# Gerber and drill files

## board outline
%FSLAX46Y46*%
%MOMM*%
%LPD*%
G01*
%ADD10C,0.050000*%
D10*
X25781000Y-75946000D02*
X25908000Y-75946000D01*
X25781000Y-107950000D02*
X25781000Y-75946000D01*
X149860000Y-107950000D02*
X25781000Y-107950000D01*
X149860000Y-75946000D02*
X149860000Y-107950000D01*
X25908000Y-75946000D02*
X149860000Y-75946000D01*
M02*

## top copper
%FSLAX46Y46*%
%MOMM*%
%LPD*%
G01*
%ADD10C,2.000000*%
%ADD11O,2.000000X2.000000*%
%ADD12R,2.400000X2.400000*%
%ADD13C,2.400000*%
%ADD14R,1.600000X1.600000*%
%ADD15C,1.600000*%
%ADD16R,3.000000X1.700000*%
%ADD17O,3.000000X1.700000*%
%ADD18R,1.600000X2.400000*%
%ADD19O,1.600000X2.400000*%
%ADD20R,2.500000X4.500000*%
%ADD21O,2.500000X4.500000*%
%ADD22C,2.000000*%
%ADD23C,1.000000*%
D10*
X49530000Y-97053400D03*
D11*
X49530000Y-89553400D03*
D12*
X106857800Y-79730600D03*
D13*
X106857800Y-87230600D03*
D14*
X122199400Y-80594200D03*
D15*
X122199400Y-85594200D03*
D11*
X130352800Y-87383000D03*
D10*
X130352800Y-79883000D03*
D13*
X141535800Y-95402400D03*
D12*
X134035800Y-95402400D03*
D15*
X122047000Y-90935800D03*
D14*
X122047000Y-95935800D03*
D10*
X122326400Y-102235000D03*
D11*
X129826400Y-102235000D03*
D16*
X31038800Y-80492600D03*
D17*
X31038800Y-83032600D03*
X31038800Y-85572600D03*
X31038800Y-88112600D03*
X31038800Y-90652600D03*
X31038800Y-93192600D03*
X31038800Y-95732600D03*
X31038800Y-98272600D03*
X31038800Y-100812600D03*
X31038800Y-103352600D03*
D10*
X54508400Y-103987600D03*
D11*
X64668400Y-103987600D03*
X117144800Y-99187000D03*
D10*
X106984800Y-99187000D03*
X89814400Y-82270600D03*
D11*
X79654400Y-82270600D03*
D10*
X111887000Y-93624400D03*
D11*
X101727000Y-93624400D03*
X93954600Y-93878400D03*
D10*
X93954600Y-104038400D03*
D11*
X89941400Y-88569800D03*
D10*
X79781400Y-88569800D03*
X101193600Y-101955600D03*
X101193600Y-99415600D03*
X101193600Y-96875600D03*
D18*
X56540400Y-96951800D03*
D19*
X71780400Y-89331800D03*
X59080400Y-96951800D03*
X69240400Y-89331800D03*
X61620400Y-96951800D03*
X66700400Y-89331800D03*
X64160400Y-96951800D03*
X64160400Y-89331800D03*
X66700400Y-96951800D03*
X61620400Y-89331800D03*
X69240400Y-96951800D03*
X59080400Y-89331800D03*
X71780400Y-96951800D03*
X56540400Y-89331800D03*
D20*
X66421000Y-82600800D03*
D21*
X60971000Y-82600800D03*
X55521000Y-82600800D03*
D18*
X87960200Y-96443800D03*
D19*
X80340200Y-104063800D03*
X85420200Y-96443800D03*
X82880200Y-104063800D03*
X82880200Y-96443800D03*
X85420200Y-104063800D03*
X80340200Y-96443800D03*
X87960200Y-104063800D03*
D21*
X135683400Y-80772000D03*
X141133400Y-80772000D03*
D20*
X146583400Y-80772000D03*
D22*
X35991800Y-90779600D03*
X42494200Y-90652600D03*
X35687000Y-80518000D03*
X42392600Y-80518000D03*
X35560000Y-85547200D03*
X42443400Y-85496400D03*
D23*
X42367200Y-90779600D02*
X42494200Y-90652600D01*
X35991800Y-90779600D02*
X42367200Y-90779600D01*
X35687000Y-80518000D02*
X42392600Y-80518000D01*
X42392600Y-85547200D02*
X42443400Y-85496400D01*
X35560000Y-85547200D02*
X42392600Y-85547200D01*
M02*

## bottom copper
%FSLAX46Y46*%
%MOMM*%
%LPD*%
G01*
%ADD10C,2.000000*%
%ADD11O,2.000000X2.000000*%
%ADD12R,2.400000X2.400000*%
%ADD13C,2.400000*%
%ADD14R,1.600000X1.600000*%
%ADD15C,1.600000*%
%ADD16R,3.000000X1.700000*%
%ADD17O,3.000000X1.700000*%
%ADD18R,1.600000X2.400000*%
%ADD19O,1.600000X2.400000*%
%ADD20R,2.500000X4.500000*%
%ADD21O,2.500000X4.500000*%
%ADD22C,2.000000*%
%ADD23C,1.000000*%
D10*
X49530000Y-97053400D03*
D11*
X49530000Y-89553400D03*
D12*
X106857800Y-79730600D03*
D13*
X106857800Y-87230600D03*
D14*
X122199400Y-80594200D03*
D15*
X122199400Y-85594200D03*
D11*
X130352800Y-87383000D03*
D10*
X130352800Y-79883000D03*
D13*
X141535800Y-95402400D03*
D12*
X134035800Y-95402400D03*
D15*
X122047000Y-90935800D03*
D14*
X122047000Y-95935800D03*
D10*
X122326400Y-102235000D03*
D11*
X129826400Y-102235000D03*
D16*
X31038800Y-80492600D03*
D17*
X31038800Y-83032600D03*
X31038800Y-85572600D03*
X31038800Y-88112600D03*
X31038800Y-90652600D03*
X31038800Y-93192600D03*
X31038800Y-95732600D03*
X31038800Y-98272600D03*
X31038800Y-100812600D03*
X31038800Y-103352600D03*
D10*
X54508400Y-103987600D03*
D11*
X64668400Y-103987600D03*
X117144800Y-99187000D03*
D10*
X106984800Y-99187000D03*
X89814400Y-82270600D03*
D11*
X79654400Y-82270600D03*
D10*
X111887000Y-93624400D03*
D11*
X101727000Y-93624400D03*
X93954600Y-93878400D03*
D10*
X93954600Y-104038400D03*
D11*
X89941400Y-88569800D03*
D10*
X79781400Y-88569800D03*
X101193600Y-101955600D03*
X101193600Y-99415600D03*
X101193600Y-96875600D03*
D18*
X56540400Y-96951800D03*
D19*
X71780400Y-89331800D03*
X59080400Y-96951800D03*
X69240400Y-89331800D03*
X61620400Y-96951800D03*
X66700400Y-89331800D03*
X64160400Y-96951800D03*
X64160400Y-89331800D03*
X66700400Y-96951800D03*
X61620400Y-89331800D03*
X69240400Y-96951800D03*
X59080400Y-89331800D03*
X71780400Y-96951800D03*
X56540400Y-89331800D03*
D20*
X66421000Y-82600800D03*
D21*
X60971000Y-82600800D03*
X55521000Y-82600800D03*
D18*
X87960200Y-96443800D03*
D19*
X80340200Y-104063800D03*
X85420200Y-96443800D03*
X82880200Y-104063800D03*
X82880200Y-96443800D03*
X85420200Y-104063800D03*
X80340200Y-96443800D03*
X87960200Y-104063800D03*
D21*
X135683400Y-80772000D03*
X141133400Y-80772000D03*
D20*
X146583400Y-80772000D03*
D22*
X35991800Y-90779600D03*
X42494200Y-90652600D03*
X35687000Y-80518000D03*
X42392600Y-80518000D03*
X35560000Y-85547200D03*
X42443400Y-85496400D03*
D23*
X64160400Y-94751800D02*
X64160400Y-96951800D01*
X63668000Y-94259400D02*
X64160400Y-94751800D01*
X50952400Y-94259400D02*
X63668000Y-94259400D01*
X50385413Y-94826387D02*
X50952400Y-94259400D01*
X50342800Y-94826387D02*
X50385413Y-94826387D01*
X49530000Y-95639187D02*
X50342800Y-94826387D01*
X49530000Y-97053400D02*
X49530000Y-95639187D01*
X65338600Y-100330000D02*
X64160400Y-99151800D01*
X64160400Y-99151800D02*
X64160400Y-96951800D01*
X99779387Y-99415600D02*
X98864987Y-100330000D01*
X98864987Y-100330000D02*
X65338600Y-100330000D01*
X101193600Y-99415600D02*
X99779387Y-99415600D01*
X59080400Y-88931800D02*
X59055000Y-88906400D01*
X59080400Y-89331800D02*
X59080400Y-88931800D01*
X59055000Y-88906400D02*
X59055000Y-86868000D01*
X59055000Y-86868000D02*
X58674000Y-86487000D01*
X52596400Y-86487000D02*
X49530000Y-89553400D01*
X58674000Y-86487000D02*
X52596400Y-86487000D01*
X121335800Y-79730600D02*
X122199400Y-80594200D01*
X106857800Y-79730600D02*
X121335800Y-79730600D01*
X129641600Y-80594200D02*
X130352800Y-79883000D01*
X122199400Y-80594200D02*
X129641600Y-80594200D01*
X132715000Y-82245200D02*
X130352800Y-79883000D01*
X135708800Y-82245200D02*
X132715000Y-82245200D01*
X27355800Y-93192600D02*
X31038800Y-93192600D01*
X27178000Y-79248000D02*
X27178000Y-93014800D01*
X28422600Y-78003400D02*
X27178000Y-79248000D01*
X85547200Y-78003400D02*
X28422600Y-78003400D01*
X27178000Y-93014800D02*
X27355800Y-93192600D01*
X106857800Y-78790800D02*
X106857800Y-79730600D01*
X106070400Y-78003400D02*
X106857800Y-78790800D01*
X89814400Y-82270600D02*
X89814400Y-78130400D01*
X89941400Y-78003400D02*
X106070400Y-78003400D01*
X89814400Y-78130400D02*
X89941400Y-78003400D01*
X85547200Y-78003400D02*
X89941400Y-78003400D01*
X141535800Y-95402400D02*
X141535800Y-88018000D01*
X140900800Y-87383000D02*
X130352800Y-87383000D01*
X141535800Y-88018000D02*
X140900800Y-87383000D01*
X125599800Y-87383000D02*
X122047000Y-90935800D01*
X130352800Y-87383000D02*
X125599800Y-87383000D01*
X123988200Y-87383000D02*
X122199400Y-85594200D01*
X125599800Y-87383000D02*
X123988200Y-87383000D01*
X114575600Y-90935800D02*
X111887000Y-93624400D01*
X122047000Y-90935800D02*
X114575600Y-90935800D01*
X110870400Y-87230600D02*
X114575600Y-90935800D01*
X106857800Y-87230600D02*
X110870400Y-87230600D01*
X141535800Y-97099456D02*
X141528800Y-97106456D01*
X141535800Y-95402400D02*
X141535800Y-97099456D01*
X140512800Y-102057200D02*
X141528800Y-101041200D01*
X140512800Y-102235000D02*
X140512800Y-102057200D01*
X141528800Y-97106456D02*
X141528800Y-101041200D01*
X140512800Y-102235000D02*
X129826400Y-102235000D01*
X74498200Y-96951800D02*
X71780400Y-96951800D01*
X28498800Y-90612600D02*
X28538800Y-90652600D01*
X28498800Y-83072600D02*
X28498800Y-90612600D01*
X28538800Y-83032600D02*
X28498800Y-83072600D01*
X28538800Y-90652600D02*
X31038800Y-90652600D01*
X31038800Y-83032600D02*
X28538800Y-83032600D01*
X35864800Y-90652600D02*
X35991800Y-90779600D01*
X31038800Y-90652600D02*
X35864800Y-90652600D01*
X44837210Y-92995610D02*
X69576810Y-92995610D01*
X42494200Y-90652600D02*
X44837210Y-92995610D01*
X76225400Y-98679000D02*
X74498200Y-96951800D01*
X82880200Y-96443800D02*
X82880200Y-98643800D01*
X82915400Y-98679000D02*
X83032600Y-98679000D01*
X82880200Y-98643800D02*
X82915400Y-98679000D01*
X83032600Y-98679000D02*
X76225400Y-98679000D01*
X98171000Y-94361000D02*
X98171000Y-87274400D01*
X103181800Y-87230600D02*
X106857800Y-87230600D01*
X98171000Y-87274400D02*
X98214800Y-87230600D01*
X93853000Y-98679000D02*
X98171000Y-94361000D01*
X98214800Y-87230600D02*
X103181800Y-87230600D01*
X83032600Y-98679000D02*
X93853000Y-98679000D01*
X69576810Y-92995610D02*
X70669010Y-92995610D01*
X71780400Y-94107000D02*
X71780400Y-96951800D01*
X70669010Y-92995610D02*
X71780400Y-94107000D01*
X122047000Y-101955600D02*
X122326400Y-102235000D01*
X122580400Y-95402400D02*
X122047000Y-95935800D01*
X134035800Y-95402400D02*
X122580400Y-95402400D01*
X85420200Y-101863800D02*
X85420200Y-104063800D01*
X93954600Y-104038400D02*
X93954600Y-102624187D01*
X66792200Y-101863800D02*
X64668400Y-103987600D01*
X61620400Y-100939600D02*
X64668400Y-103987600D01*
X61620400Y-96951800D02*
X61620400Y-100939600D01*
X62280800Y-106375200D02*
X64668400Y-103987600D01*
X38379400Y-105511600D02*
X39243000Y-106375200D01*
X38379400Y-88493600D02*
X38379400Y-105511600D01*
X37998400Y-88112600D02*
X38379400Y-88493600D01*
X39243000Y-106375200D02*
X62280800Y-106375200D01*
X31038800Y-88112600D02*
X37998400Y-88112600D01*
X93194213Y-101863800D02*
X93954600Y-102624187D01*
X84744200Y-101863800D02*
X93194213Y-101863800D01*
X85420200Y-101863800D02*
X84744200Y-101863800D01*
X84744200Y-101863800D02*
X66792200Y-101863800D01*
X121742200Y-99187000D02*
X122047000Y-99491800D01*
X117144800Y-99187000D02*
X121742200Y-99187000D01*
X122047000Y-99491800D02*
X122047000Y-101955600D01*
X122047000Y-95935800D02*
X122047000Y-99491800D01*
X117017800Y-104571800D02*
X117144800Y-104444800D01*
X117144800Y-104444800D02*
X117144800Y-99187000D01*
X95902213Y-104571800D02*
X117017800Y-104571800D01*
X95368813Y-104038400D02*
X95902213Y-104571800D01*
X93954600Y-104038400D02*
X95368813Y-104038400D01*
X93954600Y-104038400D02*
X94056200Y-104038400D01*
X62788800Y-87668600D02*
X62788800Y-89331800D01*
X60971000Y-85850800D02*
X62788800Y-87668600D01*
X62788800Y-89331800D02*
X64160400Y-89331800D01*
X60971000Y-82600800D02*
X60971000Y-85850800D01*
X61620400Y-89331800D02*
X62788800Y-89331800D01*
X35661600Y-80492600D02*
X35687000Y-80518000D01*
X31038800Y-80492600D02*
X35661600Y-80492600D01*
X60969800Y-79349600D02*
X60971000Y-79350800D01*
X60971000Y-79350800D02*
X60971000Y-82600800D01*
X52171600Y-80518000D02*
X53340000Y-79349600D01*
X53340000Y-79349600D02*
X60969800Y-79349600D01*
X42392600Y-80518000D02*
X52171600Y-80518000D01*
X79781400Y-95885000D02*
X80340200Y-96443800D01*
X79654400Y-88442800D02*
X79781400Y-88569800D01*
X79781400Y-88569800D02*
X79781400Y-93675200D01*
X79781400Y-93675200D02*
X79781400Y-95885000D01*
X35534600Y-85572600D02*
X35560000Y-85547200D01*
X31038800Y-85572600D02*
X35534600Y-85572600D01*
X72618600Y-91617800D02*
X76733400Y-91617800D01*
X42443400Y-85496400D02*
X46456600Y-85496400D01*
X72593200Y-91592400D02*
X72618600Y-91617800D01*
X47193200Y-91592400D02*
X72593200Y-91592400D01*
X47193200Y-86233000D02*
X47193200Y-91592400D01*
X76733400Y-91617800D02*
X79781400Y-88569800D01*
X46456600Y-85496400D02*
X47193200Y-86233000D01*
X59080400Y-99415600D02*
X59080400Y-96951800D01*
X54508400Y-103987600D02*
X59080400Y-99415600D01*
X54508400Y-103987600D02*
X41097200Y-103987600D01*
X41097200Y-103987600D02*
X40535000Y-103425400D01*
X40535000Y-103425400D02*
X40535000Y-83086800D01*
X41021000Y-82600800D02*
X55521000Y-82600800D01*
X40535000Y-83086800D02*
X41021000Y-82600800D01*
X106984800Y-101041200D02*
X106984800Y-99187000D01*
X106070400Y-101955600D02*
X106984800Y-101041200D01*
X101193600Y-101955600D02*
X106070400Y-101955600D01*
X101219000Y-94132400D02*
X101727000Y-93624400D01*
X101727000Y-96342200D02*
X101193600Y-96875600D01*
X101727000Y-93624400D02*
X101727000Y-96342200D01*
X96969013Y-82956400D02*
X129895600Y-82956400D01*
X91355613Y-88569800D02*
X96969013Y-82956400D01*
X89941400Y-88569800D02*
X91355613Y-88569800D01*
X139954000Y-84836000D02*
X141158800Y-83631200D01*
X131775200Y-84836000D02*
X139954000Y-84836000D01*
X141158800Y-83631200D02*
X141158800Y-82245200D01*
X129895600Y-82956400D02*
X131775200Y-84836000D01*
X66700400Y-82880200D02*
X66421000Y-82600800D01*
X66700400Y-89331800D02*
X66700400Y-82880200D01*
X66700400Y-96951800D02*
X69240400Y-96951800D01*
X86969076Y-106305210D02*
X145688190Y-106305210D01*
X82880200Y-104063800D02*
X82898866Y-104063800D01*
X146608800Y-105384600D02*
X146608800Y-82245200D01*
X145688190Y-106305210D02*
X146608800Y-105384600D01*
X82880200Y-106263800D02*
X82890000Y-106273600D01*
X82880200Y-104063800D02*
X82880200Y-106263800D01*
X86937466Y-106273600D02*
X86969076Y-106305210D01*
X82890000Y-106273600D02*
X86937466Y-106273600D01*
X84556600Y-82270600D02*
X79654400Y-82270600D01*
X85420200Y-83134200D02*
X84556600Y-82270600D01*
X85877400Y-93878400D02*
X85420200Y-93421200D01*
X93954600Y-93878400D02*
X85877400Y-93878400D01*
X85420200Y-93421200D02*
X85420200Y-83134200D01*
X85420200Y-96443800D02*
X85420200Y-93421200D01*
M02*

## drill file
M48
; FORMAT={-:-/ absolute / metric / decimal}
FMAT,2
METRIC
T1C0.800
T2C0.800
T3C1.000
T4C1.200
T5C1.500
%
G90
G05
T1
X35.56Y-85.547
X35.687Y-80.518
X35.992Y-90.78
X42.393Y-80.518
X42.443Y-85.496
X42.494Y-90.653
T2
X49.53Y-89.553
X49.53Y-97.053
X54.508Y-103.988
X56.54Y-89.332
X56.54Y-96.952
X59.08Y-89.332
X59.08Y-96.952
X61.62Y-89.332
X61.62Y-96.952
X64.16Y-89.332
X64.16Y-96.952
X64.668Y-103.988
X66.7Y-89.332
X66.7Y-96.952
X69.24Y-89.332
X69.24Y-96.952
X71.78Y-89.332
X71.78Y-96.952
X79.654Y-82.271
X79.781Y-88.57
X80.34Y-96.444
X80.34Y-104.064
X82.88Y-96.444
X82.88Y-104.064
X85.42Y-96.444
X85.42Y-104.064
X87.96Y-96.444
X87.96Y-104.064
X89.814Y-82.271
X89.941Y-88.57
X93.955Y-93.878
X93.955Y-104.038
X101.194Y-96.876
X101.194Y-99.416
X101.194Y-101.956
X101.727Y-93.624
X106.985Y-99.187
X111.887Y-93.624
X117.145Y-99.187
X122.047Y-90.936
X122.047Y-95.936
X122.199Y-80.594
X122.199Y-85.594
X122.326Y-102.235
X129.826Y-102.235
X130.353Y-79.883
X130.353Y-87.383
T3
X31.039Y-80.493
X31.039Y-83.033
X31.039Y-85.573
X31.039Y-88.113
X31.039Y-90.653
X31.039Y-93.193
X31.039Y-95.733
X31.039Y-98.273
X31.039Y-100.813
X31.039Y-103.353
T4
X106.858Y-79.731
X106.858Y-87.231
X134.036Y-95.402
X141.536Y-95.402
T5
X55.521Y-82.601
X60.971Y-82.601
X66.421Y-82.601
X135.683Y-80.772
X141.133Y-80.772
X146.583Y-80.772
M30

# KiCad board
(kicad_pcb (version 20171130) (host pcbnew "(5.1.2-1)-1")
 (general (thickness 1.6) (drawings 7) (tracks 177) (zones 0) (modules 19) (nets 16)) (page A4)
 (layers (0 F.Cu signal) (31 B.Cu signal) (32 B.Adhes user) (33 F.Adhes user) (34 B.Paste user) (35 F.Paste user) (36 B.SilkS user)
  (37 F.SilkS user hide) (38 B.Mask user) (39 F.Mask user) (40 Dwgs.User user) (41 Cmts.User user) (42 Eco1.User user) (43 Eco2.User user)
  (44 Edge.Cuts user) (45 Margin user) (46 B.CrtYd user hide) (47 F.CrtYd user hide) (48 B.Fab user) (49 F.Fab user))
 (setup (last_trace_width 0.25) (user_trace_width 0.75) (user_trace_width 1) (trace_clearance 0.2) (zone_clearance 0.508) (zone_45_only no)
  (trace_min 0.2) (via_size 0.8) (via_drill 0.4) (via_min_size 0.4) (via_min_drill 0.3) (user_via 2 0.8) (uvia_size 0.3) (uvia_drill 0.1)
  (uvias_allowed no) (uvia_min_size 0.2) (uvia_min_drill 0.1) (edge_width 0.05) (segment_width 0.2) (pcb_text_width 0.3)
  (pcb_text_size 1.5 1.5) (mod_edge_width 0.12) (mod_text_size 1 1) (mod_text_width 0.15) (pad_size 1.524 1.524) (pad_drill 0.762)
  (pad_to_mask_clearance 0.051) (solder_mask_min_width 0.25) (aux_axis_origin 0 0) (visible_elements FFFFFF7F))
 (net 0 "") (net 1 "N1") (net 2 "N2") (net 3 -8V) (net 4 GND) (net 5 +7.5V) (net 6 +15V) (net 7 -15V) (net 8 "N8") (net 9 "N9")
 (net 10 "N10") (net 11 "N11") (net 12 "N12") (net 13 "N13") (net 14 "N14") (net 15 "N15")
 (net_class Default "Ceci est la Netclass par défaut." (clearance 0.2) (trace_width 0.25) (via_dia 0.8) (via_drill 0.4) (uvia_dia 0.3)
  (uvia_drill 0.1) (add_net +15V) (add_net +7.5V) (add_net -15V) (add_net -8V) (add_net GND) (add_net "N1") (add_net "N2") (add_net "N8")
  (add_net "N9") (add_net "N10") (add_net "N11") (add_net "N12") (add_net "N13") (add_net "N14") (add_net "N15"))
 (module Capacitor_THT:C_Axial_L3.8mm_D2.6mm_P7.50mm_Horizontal (layer F.Cu) (at 49.53 97.0534 90)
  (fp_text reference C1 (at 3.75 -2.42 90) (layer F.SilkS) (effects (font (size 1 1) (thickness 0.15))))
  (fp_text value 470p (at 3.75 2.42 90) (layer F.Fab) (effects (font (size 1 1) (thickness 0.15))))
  (pad 1 thru_hole circle (at 0 0 90) (size 2 2) (drill 0.8) (layers *.Cu *.Mask) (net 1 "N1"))
  (pad 2 thru_hole oval (at 7.5 0 90) (size 2 2) (drill 0.8) (layers *.Cu *.Mask) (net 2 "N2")))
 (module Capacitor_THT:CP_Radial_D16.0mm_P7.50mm (layer F.Cu) (at 106.8578 79.7306 270)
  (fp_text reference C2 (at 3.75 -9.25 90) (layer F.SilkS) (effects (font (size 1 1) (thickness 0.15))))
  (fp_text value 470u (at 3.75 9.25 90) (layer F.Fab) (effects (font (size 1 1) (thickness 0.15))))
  (pad 1 thru_hole rect (at 0 0 270) (size 2.4 2.4) (drill 1.2) (layers *.Cu *.Mask) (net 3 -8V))
  (pad 2 thru_hole circle (at 7.5 0 270) (size 2.4 2.4) (drill 1.2) (layers *.Cu *.Mask) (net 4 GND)))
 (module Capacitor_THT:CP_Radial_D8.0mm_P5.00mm (layer F.Cu) (at 122.1994 80.5942 270)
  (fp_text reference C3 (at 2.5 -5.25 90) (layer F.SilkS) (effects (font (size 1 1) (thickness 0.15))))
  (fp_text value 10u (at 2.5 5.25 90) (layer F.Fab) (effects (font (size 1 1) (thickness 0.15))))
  (pad 1 thru_hole rect (at 0 0 270) (size 1.6 1.6) (drill 0.8) (layers *.Cu *.Mask) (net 3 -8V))
  (pad 2 thru_hole circle (at 5 0 270) (size 1.6 1.6) (drill 0.8) (layers *.Cu *.Mask) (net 4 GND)))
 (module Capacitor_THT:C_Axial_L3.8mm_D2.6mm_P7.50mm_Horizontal (layer F.Cu) (at 130.3528 79.883 270)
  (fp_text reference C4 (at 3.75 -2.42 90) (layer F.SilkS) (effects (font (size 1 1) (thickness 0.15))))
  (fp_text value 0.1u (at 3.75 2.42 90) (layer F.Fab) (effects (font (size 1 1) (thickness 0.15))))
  (pad 2 thru_hole oval (at 7.5 0 270) (size 2 2) (drill 0.8) (layers *.Cu *.Mask) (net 4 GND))
  (pad 1 thru_hole circle (at 0 0 270) (size 2 2) (drill 0.8) (layers *.Cu *.Mask) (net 3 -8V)))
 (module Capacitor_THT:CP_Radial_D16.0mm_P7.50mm (layer F.Cu) (at 134.0358 95.4024)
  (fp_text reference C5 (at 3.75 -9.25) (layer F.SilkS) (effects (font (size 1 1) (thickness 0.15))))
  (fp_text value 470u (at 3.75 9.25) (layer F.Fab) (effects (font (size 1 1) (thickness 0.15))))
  (pad 2 thru_hole circle (at 7.5 0) (size 2.4 2.4) (drill 1.2) (layers *.Cu *.Mask) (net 4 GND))
  (pad 1 thru_hole rect (at 0 0) (size 2.4 2.4) (drill 1.2) (layers *.Cu *.Mask) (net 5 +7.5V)))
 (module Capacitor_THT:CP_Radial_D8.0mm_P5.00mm (layer F.Cu) (at 122.047 95.9358 90)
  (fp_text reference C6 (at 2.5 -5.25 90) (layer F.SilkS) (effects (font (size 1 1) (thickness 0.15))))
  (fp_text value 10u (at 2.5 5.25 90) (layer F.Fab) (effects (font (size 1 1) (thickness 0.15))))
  (pad 2 thru_hole circle (at 5 0 90) (size 1.6 1.6) (drill 0.8) (layers *.Cu *.Mask) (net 4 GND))
  (pad 1 thru_hole rect (at 0 0 90) (size 1.6 1.6) (drill 0.8) (layers *.Cu *.Mask) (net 5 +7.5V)))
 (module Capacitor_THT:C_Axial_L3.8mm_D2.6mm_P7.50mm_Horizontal (layer F.Cu) (at 122.3264 102.235)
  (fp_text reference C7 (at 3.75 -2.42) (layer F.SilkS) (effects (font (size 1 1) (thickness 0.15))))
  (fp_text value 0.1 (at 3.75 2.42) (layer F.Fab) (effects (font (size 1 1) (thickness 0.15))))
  (pad 1 thru_hole circle (at 0 0) (size 2 2) (drill 0.8) (layers *.Cu *.Mask) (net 5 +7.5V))
  (pad 2 thru_hole oval (at 7.5 0) (size 2 2) (drill 0.8) (layers *.Cu *.Mask) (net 4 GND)))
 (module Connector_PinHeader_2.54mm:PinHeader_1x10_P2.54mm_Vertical (layer F.Cu) (at 31.0388 80.4926)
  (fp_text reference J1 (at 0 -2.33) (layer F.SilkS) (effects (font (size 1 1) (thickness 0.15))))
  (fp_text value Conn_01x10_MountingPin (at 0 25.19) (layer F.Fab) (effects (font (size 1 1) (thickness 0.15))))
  (pad 1 thru_hole rect (at 0 0) (size 3 1.7) (drill 1) (layers *.Cu *.Mask) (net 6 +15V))
  (pad 2 thru_hole oval (at 0 2.54) (size 3 1.7) (drill 1) (layers *.Cu *.Mask) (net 4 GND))
  (pad 3 thru_hole oval (at 0 5.08) (size 3 1.7) (drill 1) (layers *.Cu *.Mask) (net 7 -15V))
  (pad 4 thru_hole oval (at 0 7.62) (size 3 1.7) (drill 1) (layers *.Cu *.Mask) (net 5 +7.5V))
  (pad 5 thru_hole oval (at 0 10.16) (size 3 1.7) (drill 1) (layers *.Cu *.Mask) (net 4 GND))
  (pad 6 thru_hole oval (at 0 12.7) (size 3 1.7) (drill 1) (layers *.Cu *.Mask) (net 3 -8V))
  (pad 7 thru_hole oval (at 0 15.24) (size 3 1.7) (drill 1) (layers *.Cu *.Mask))
  (pad 8 thru_hole oval (at 0 17.78) (size 3 1.7) (drill 1) (layers *.Cu *.Mask))
  (pad 9 thru_hole oval (at 0 20.32) (size 3 1.7) (drill 1) (layers *.Cu *.Mask))
  (pad 10 thru_hole oval (at 0 22.86) (size 3 1.7) (drill 1) (layers *.Cu *.Mask)))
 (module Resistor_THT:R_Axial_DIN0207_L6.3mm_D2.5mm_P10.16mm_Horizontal (layer F.Cu) (at 54.5084 103.9876)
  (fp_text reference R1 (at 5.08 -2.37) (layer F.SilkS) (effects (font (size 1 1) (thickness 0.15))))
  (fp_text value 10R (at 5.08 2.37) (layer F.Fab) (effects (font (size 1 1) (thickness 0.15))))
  (pad 1 thru_hole circle (at 0 0) (size 2 2) (drill 0.8) (layers *.Cu *.Mask) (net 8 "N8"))
  (pad 2 thru_hole oval (at 10.16 0) (size 2 2) (drill 0.8) (layers *.Cu *.Mask) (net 5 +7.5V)))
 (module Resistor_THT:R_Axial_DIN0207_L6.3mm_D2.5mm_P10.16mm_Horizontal (layer F.Cu) (at 106.9848 99.187)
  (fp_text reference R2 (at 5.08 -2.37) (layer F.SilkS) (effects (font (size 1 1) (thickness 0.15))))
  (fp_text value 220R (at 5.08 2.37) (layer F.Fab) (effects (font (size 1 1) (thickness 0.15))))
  (pad 2 thru_hole oval (at 10.16 0) (size 2 2) (drill 0.8) (layers *.Cu *.Mask) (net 5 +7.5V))
  (pad 1 thru_hole circle (at 0 0) (size 2 2) (drill 0.8) (layers *.Cu *.Mask) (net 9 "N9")))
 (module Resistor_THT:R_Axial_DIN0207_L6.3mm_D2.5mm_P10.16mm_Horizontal (layer F.Cu) (at 89.8144 82.2706 180)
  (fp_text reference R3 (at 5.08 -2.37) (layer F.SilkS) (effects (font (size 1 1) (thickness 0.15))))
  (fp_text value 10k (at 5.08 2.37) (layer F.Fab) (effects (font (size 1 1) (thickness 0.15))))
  (pad 1 thru_hole circle (at 0 0 180) (size 2 2) (drill 0.8) (layers *.Cu *.Mask) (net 3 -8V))
  (pad 2 thru_hole oval (at 10.16 0 180) (size 2 2) (drill 0.8) (layers *.Cu *.Mask) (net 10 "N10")))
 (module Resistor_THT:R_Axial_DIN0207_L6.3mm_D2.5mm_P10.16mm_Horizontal (layer F.Cu) (at 111.887 93.6244 180)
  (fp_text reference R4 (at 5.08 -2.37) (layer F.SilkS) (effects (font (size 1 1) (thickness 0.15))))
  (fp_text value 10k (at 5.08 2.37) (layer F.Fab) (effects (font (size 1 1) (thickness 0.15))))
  (pad 1 thru_hole circle (at 0 0 180) (size 2 2) (drill 0.8) (layers *.Cu *.Mask) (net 4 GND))
  (pad 2 thru_hole oval (at 10.16 0 180) (size 2 2) (drill 0.8) (layers *.Cu *.Mask) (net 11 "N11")))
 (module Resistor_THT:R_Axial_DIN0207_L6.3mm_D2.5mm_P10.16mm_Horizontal (layer F.Cu) (at 93.9546 104.0384 90)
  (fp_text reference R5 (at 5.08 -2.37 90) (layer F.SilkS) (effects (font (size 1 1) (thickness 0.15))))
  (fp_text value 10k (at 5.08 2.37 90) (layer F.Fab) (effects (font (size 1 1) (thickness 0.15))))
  (pad 2 thru_hole oval (at 10.16 0 90) (size 2 2) (drill 0.8) (layers *.Cu *.Mask) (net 10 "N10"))
  (pad 1 thru_hole circle (at 0 0 90) (size 2 2) (drill 0.8) (layers *.Cu *.Mask) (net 5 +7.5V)))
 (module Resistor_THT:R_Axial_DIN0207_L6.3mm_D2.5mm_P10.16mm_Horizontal (layer F.Cu) (at 79.7814 88.5698)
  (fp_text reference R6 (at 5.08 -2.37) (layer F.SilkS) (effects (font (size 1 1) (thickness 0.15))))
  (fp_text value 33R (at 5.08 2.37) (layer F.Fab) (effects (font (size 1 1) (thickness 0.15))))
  (pad 2 thru_hole oval (at 10.16 0) (size 2 2) (drill 0.8) (layers *.Cu *.Mask) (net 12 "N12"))
  (pad 1 thru_hole circle (at 0 0) (size 2 2) (drill 0.8) (layers *.Cu *.Mask) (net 7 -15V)))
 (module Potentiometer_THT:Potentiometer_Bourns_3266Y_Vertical (layer F.Cu) (at 101.1936 101.9556 270)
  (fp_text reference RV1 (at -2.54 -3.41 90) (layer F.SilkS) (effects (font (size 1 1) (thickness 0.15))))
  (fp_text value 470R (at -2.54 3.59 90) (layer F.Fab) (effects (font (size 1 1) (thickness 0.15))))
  (pad 1 thru_hole circle (at 0 0 270) (size 2 2) (drill 0.8) (layers *.Cu *.Mask) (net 9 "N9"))
  (pad 2 thru_hole circle (at -2.54 0 270) (size 2 2) (drill 0.8) (layers *.Cu *.Mask) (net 1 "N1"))
  (pad 3 thru_hole circle (at -5.08 0 270) (size 2 2) (drill 0.8) (layers *.Cu *.Mask) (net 11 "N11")))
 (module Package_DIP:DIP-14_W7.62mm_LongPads (layer F.Cu) (at 56.5404 96.9518 90)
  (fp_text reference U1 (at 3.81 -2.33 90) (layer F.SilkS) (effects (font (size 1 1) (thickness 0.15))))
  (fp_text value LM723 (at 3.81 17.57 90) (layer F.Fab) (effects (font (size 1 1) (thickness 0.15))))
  (pad 1 thru_hole rect (at 0 0 90) (size 2.4 1.6) (drill 0.8) (layers *.Cu *.Mask))
  (pad 8 thru_hole oval (at 7.62 15.24 90) (size 2.4 1.6) (drill 0.8) (layers *.Cu *.Mask))
  (pad 2 thru_hole oval (at 0 2.54 90) (size 2.4 1.6) (drill 0.8) (layers *.Cu *.Mask) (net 8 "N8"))
  (pad 9 thru_hole oval (at 7.62 12.7 90) (size 2.4 1.6) (drill 0.8) (layers *.Cu *.Mask))
  (pad 3 thru_hole oval (at 0 5.08 90) (size 2.4 1.6) (drill 0.8) (layers *.Cu *.Mask) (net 5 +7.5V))
  (pad 10 thru_hole oval (at 7.62 10.16 90) (size 2.4 1.6) (drill 0.8) (layers *.Cu *.Mask) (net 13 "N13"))
  (pad 4 thru_hole oval (at 0 7.62 90) (size 2.4 1.6) (drill 0.8) (layers *.Cu *.Mask) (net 1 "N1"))
  (pad 11 thru_hole oval (at 7.62 7.62 90) (size 2.4 1.6) (drill 0.8) (layers *.Cu *.Mask) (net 6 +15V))
  (pad 5 thru_hole oval (at 0 10.16 90) (size 2.4 1.6) (drill 0.8) (layers *.Cu *.Mask) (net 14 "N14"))
  (pad 12 thru_hole oval (at 7.62 5.08 90) (size 2.4 1.6) (drill 0.8) (layers *.Cu *.Mask) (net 6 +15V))
  (pad 6 thru_hole oval (at 0 12.7 90) (size 2.4 1.6) (drill 0.8) (layers *.Cu *.Mask) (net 14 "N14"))
  (pad 13 thru_hole oval (at 7.62 2.54 90) (size 2.4 1.6) (drill 0.8) (layers *.Cu *.Mask) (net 2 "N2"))
  (pad 7 thru_hole oval (at 0 15.24 90) (size 2.4 1.6) (drill 0.8) (layers *.Cu *.Mask) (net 4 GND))
  (pad 14 thru_hole oval (at 7.62 0 90) (size 2.4 1.6) (drill 0.8) (layers *.Cu *.Mask)))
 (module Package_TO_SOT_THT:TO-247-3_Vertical (layer F.Cu) (at 66.421 82.6008 180)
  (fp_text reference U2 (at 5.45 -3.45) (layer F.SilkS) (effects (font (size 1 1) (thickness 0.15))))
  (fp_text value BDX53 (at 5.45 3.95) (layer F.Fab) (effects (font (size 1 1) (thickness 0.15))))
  (pad 1 thru_hole rect (at 0 0 180) (size 2.5 4.5) (drill 1.5) (layers *.Cu *.Mask) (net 13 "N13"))
  (pad 2 thru_hole oval (at 5.45 0 180) (size 2.5 4.5) (drill 1.5) (layers *.Cu *.Mask) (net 6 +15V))
  (pad 3 thru_hole oval (at 10.9 0 180) (size 2.5 4.5) (drill 1.5) (layers *.Cu *.Mask) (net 8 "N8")))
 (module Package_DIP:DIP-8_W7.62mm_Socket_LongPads (layer F.Cu) (at 87.9602 96.4438 270)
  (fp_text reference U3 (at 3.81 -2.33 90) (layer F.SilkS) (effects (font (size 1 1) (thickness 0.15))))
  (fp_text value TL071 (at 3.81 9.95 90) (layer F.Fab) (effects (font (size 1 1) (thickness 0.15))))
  (pad 1 thru_hole rect (at 0 0 270) (size 2.4 1.6) (drill 0.8) (layers *.Cu *.Mask))
  (pad 5 thru_hole oval (at 7.62 7.62 270) (size 2.4 1.6) (drill 0.8) (layers *.Cu *.Mask))
  (pad 2 thru_hole oval (at 0 2.54 270) (size 2.4 1.6) (drill 0.8) (layers *.Cu *.Mask) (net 10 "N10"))
  (pad 6 thru_hole oval (at 7.62 5.08 270) (size 2.4 1.6) (drill 0.8) (layers *.Cu *.Mask) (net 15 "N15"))
  (pad 3 thru_hole oval (at 0 5.08 270) (size 2.4 1.6) (drill 0.8) (layers *.Cu *.Mask) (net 4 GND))
  (pad 7 thru_hole oval (at 7.62 2.54 270) (size 2.4 1.6) (drill 0.8) (layers *.Cu *.Mask) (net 5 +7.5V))
  (pad 4 thru_hole oval (at 0 7.62 270) (size 2.4 1.6) (drill 0.8) (layers *.Cu *.Mask) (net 7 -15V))
  (pad 8 thru_hole oval (at 7.62 0 270) (size 2.4 1.6) (drill 0.8) (layers *.Cu *.Mask)))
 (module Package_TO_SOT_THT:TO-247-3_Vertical (layer F.Cu) (at 146.5834 80.772 180)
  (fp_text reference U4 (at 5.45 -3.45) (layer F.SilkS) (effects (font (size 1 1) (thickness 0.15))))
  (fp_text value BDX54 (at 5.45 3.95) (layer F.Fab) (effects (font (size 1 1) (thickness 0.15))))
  (pad 3 thru_hole oval (at 10.9 0 180) (size 2.5 4.5) (drill 1.5) (layers *.Cu *.Mask) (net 3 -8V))
  (pad 2 thru_hole oval (at 5.45 0 180) (size 2.5 4.5) (drill 1.5) (layers *.Cu *.Mask) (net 12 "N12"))
  (pad 1 thru_hole rect (at 0 0 180) (size 2.5 4.5) (drill 1.5) (layers *.Cu *.Mask) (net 15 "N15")))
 (gr_line (start 25.781 75.946) (end 25.908 75.946) (layer Edge.Cuts) (width 0.05))
 (gr_line (start 25.781 107.95) (end 25.781 75.946) (layer Edge.Cuts) (width 0.05))
 (gr_line (start 149.86 107.95) (end 25.781 107.95) (layer Edge.Cuts) (width 0.05))
 (gr_line (start 149.86 75.946) (end 149.86 107.95) (layer Edge.Cuts) (width 0.05))
 (gr_line (start 25.908 75.946) (end 149.86 75.946) (layer Edge.Cuts) (width 0.05))
 (segment (start 64.1604 94.7518) (end 64.1604 96.9518) (width 1) (layer B.Cu) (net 1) (status 20))
 (segment (start 63.668 94.2594) (end 64.1604 94.7518) (width 1) (layer B.Cu) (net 1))
 (segment (start 50.9524 94.2594) (end 63.668 94.2594) (width 1) (layer B.Cu) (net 1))
 (segment (start 50.385413 94.826387) (end 50.9524 94.2594) (width 1) (layer B.Cu) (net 1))
 (segment (start 50.3428 94.826387) (end 50.385413 94.826387) (width 1) (layer B.Cu) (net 1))
 (segment (start 49.53 95.639187) (end 50.3428 94.826387) (width 1) (layer B.Cu) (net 1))
 (segment (start 49.53 97.0534) (end 49.53 95.639187) (width 1) (layer B.Cu) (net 1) (status 10))
 (segment (start 65.3386 100.33) (end 64.1604 99.1518) (width 1) (layer B.Cu) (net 1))
 (segment (start 64.1604 99.1518) (end 64.1604 96.9518) (width 1) (layer B.Cu) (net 1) (status 20))
 (segment (start 99.779387 99.4156) (end 98.864987 100.33) (width 1) (layer B.Cu) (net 1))
 (segment (start 98.864987 100.33) (end 65.3386 100.33) (width 1) (layer B.Cu) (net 1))
 (segment (start 101.1936 99.4156) (end 99.779387 99.4156) (width 1) (layer B.Cu) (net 1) (status 10))
 (segment (start 59.0804 88.9318) (end 59.055 88.9064) (width 1) (layer B.Cu) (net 2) (status 30))
 (segment (start 59.0804 89.3318) (end 59.0804 88.9318) (width 1) (layer B.Cu) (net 2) (status 30))
 (segment (start 59.055 88.9064) (end 59.055 86.868) (width 1) (layer B.Cu) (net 2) (status 10))
 (segment (start 59.055 86.868) (end 58.674 86.487) (width 1) (layer B.Cu) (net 2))
 (segment (start 52.5964 86.487) (end 49.53 89.5534) (width 1) (layer B.Cu) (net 2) (status 20))
 (segment (start 58.674 86.487) (end 52.5964 86.487) (width 1) (layer B.Cu) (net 2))
 (segment (start 121.3358 79.7306) (end 122.1994 80.5942) (width 1) (layer B.Cu) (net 3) (status 20))
 (segment (start 106.8578 79.7306) (end 121.3358 79.7306) (width 1) (layer B.Cu) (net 3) (status 10))
 (segment (start 129.6416 80.5942) (end 130.3528 79.883) (width 1) (layer B.Cu) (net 3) (status 20))
 (segment (start 122.1994 80.5942) (end 129.6416 80.5942) (width 1) (layer B.Cu) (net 3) (status 10))
 (segment (start 132.715 82.2452) (end 130.3528 79.883) (width 1) (layer B.Cu) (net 3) (status 20))
 (segment (start 135.7088 82.2452) (end 132.715 82.2452) (width 1) (layer B.Cu) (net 3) (status 10))
 (segment (start 27.3558 93.1926) (end 31.0388 93.1926) (width 1) (layer B.Cu) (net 3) (status 20))
 (segment (start 27.178 79.248) (end 27.178 93.0148) (width 1) (layer B.Cu) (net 3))
 (segment (start 28.4226 78.0034) (end 27.178 79.248) (width 1) (layer B.Cu) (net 3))
 (segment (start 85.5472 78.0034) (end 28.4226 78.0034) (width 1) (layer B.Cu) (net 3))
 (segment (start 27.178 93.0148) (end 27.3558 93.1926) (width 1) (layer B.Cu) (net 3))
 (segment (start 106.8578 78.7908) (end 106.8578 79.7306) (width 1) (layer B.Cu) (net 3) (status 30))
 (segment (start 106.0704 78.0034) (end 106.8578 78.7908) (width 1) (layer B.Cu) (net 3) (status 20))
 (segment (start 89.8144 82.2706) (end 89.8144 78.1304) (width 1) (layer B.Cu) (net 3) (status 10))
 (segment (start 89.9414 78.0034) (end 106.0704 78.0034) (width 1) (layer B.Cu) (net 3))
 (segment (start 89.8144 78.1304) (end 89.9414 78.0034) (width 1) (layer B.Cu) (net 3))
 (segment (start 85.5472 78.0034) (end 89.9414 78.0034) (width 1) (layer B.Cu) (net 3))
 (segment (start 141.5358 95.4024) (end 141.5358 88.018) (width 1) (layer B.Cu) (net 4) (status 10))
 (segment (start 140.9008 87.383) (end 130.3528 87.383) (width 1) (layer B.Cu) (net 4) (status 20))
 (segment (start 141.5358 88.018) (end 140.9008 87.383) (width 1) (layer B.Cu) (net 4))
 (segment (start 125.5998 87.383) (end 122.047 90.9358) (width 1) (layer B.Cu) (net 4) (status 20))
 (segment (start 130.3528 87.383) (end 125.5998 87.383) (width 1) (layer B.Cu) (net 4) (status 10))
 (segment (start 123.9882 87.383) (end 122.1994 85.5942) (width 1) (layer B.Cu) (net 4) (status 20))
 (segment (start 125.5998 87.383) (end 123.9882 87.383) (width 1) (layer B.Cu) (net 4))
 (segment (start 114.5756 90.9358) (end 111.887 93.6244) (width 1) (layer B.Cu) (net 4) (status 20))
 (segment (start 122.047 90.9358) (end 114.5756 90.9358) (width 1) (layer B.Cu) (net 4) (status 10))
 (segment (start 110.8704 87.2306) (end 114.5756 90.9358) (width 1) (layer B.Cu) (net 4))
 (segment (start 106.8578 87.2306) (end 110.8704 87.2306) (width 1) (layer B.Cu) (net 4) (status 10))
 (segment (start 141.5358 97.099456) (end 141.5288 97.106456) (width 1) (layer B.Cu) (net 4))
 (segment (start 141.5358 95.4024) (end 141.5358 97.099456) (width 1) (layer B.Cu) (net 4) (status 10))
 (segment (start 140.5128 102.0572) (end 141.5288 101.0412) (width 1) (layer B.Cu) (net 4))
 (segment (start 140.5128 102.235) (end 140.5128 102.0572) (width 1) (layer B.Cu) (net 4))
 (segment (start 141.5288 97.106456) (end 141.5288 101.0412) (width 1) (layer B.Cu) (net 4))
 (segment (start 140.5128 102.235) (end 129.8264 102.235) (width 1) (layer B.Cu) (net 4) (status 20))
 (segment (start 74.4982 96.9518) (end 71.7804 96.9518) (width 1) (layer B.Cu) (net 4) (status 20))
 (segment (start 28.4988 90.6126) (end 28.5388 90.6526) (width 1) (layer B.Cu) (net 4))
 (segment (start 28.4988 83.0726) (end 28.4988 90.6126) (width 1) (layer B.Cu) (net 4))
 (segment (start 28.5388 83.0326) (end 28.4988 83.0726) (width 1) (layer B.Cu) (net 4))
 (segment (start 28.5388 90.6526) (end 31.0388 90.6526) (width 1) (layer B.Cu) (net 4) (status 20))
 (segment (start 31.0388 83.0326) (end 28.5388 83.0326) (width 1) (layer B.Cu) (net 4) (status 10))
 (via (at 35.9918 90.7796) (size 2) (drill 0.8) (layers F.Cu B.Cu) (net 4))
 (segment (start 35.8648 90.6526) (end 35.9918 90.7796) (width 1) (layer B.Cu) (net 4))
 (segment (start 31.0388 90.6526) (end 35.8648 90.6526) (width 1) (layer B.Cu) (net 4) (status 10))
 (via (at 42.4942 90.6526) (size 2) (drill 0.8) (layers F.Cu B.Cu) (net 4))
 (segment (start 42.3672 90.7796) (end 42.4942 90.6526) (width 1) (layer F.Cu) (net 4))
 (segment (start 35.9918 90.7796) (end 42.3672 90.7796) (width 1) (layer F.Cu) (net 4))
 (segment (start 44.83721 92.99561) (end 69.57681 92.99561) (width 1) (layer B.Cu) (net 4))
 (segment (start 42.4942 90.6526) (end 44.83721 92.99561) (width 1) (layer B.Cu) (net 4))
 (segment (start 76.2254 98.679) (end 74.4982 96.9518) (width 1) (layer B.Cu) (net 4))
 (segment (start 82.8802 96.4438) (end 82.8802 98.6438) (width 1) (layer B.Cu) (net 4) (status 10))
 (segment (start 82.9154 98.679) (end 83.0326 98.679) (width 1) (layer B.Cu) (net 4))
 (segment (start 82.8802 98.6438) (end 82.9154 98.679) (width 1) (layer B.Cu) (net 4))
 (segment (start 83.0326 98.679) (end 76.2254 98.679) (width 1) (layer B.Cu) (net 4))
 (segment (start 98.171 94.361) (end 98.171 87.2744) (width 1) (layer B.Cu) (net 4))
 (segment (start 103.1818 87.2306) (end 106.8578 87.2306) (width 1) (layer B.Cu) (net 4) (status 20))
 (segment (start 98.171 87.2744) (end 98.2148 87.2306) (width 1) (layer B.Cu) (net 4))
 (segment (start 93.853 98.679) (end 98.171 94.361) (width 1) (layer B.Cu) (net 4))
 (segment (start 98.2148 87.2306) (end 103.1818 87.2306) (width 1) (layer B.Cu) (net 4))
 (segment (start 83.0326 98.679) (end 93.853 98.679) (width 1) (layer B.Cu) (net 4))
 (segment (start 69.57681 92.99561) (end 70.66901 92.99561) (width 1) (layer B.Cu) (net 4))
 (segment (start 71.7804 94.107) (end 71.7804 96.9518) (width 1) (layer B.Cu) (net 4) (status 20))
 (segment (start 70.66901 92.99561) (end 71.7804 94.107) (width 1) (layer B.Cu) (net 4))
 (segment (start 122.047 101.9556) (end 122.3264 102.235) (width 1) (layer B.Cu) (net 5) (status 30))
 (segment (start 122.5804 95.4024) (end 122.047 95.9358) (width 1) (layer B.Cu) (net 5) (status 30))
 (segment (start 134.0358 95.4024) (end 122.5804 95.4024) (width 1) (layer B.Cu) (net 5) (status 30))
 (segment (start 85.4202 101.8638) (end 85.4202 104.0638) (width 1) (layer B.Cu) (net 5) (status 20))
 (segment (start 93.9546 104.0384) (end 93.9546 102.624187) (width 1) (layer B.Cu) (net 5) (status 10))
 (segment (start 66.7922 101.8638) (end 64.6684 103.9876) (width 1) (layer B.Cu) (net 5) (status 20))
 (segment (start 61.6204 100.9396) (end 64.6684 103.9876) (width 1) (layer B.Cu) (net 5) (status 20))
 (segment (start 61.6204 96.9518) (end 61.6204 100.9396) (width 1) (layer B.Cu) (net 5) (status 10))
 (segment (start 62.2808 106.3752) (end 64.6684 103.9876) (width 1) (layer B.Cu) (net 5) (status 20))
 (segment (start 38.3794 105.5116) (end 39.243 106.3752) (width 1) (layer B.Cu) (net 5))
 (segment (start 38.3794 88.4936) (end 38.3794 105.5116) (width 1) (layer B.Cu) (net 5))
 (segment (start 37.9984 88.1126) (end 38.3794 88.4936) (width 1) (layer B.Cu) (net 5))
 (segment (start 39.243 106.3752) (end 62.2808 106.3752) (width 1) (layer B.Cu) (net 5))
 (segment (start 31.0388 88.1126) (end 37.9984 88.1126) (width 1) (layer B.Cu) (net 5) (status 10))
 (segment (start 93.194213 101.8638) (end 93.9546 102.624187) (width 1) (layer B.Cu) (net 5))
 (segment (start 84.7442 101.8638) (end 93.194213 101.8638) (width 1) (layer B.Cu) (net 5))
 (segment (start 85.4202 101.8638) (end 84.7442 101.8638) (width 1) (layer B.Cu) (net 5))
 (segment (start 84.7442 101.8638) (end 66.7922 101.8638) (width 1) (layer B.Cu) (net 5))
 (segment (start 121.7422 99.187) (end 122.047 99.4918) (width 1) (layer B.Cu) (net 5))
 (segment (start 117.1448 99.187) (end 121.7422 99.187) (width 1) (layer B.Cu) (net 5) (status 10))
 (segment (start 122.047 99.4918) (end 122.047 101.9556) (width 1) (layer B.Cu) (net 5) (status 20))
 (segment (start 122.047 95.9358) (end 122.047 99.4918) (width 1) (layer B.Cu) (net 5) (status 10))
 (segment (start 117.0178 104.5718) (end 117.1448 104.4448) (width 1) (layer B.Cu) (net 5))
 (segment (start 117.1448 104.4448) (end 117.1448 99.187) (width 1) (layer B.Cu) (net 5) (status 20))
 (segment (start 95.902213 104.5718) (end 117.0178 104.5718) (width 1) (layer B.Cu) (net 5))
 (segment (start 95.368813 104.0384) (end 95.902213 104.5718) (width 1) (layer B.Cu) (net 5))
 (segment (start 93.9546 104.0384) (end 95.368813 104.0384) (width 1) (layer B.Cu) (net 5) (status 10))
 (segment (start 93.9546 104.0384) (end 94.0562 104.0384) (width 1) (layer B.Cu) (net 5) (status 30))
 (segment (start 62.7888 87.6686) (end 62.7888 89.3318) (width 1) (layer B.Cu) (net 6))
 (segment (start 60.971 85.8508) (end 62.7888 87.6686) (width 1) (layer B.Cu) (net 6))
 (segment (start 62.7888 89.3318) (end 64.1604 89.3318) (width 1) (layer B.Cu) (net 6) (status 20))
 (segment (start 60.971 82.6008) (end 60.971 85.8508) (width 1) (layer B.Cu) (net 6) (status 10))
 (segment (start 61.6204 89.3318) (end 62.7888 89.3318) (width 1) (layer B.Cu) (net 6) (status 10))
 (via (at 35.687 80.518) (size 2) (drill 0.8) (layers F.Cu B.Cu) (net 6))
 (segment (start 35.6616 80.4926) (end 35.687 80.518) (width 1) (layer B.Cu) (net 6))
 (segment (start 31.0388 80.4926) (end 35.6616 80.4926) (width 1) (layer B.Cu) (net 6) (status 10))
 (via (at 42.3926 80.518) (size 2) (drill 0.8) (layers F.Cu B.Cu) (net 6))
 (segment (start 35.687 80.518) (end 42.3926 80.518) (width 1) (layer F.Cu) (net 6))
 (segment (start 60.9698 79.3496) (end 60.971 79.3508) (width 1) (layer B.Cu) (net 6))
 (segment (start 60.971 79.3508) (end 60.971 82.6008) (width 1) (layer B.Cu) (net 6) (status 20))
 (segment (start 52.1716 80.518) (end 53.34 79.3496) (width 1) (layer B.Cu) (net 6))
 (segment (start 53.34 79.3496) (end 60.9698 79.3496) (width 1) (layer B.Cu) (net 6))
 (segment (start 42.3926 80.518) (end 52.1716 80.518) (width 1) (layer B.Cu) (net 6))
 (segment (start 79.7814 95.885) (end 80.3402 96.4438) (width 1) (layer B.Cu) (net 7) (status 30))
 (segment (start 79.6544 88.4428) (end 79.7814 88.5698) (width 1) (layer B.Cu) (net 7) (status 30))
 (segment (start 79.7814 88.5698) (end 79.7814 93.6752) (width 1) (layer B.Cu) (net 7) (status 10))
 (segment (start 79.7814 93.6752) (end 79.7814 95.885) (width 1) (layer B.Cu) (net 7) (status 20))
 (via (at 35.56 85.5472) (size 2) (drill 0.8) (layers F.Cu B.Cu) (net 7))
 (segment (start 35.5346 85.5726) (end 35.56 85.5472) (width 1) (layer B.Cu) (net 7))
 (segment (start 31.0388 85.5726) (end 35.5346 85.5726) (width 1) (layer B.Cu) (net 7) (status 10))
 (via (at 42.4434 85.4964) (size 2) (drill 0.8) (layers F.Cu B.Cu) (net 7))
 (segment (start 42.3926 85.5472) (end 42.4434 85.4964) (width 1) (layer F.Cu) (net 7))
 (segment (start 35.56 85.5472) (end 42.3926 85.5472) (width 1) (layer F.Cu) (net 7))
 (segment (start 72.6186 91.6178) (end 76.7334 91.6178) (width 1) (layer B.Cu) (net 7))
 (segment (start 42.4434 85.4964) (end 46.4566 85.4964) (width 1) (layer B.Cu) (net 7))
 (segment (start 72.5932 91.5924) (end 72.6186 91.6178) (width 1) (layer B.Cu) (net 7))
 (segment (start 47.1932 91.5924) (end 72.5932 91.5924) (width 1) (layer B.Cu) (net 7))
 (segment (start 47.1932 86.233) (end 47.1932 91.5924) (width 1) (layer B.Cu) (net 7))
 (segment (start 76.7334 91.6178) (end 79.7814 88.5698) (width 1) (layer B.Cu) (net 7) (status 20))
 (segment (start 46.4566 85.4964) (end 47.1932 86.233) (width 1) (layer B.Cu) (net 7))
 (segment (start 59.0804 99.4156) (end 59.0804 96.9518) (width 1) (layer B.Cu) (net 8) (status 20))
 (segment (start 54.5084 103.9876) (end 59.0804 99.4156) (width 1) (layer B.Cu) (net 8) (status 10))
 (segment (start 54.5084 103.9876) (end 41.0972 103.9876) (width 1) (layer B.Cu) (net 8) (status 10))
 (segment (start 41.0972 103.9876) (end 40.535 103.4254) (width 1) (layer B.Cu) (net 8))
 (segment (start 40.535 103.4254) (end 40.535 83.0868) (width 1) (layer B.Cu) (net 8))
 (segment (start 41.021 82.6008) (end 55.521 82.6008) (width 1) (layer B.Cu) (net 8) (status 20))
 (segment (start 40.535 83.0868) (end 41.021 82.6008) (width 1) (layer B.Cu) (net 8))
 (segment (start 106.9848 101.0412) (end 106.9848 99.187) (width 1) (layer B.Cu) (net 9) (status 20))
 (segment (start 106.0704 101.9556) (end 106.9848 101.0412) (width 1) (layer B.Cu) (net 9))
 (segment (start 101.1936 101.9556) (end 106.0704 101.9556) (width 1) (layer B.Cu) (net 9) (status 10))
 (segment (start 101.219 94.1324) (end 101.727 93.6244) (width 1) (layer B.Cu) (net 11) (status 30))
 (segment (start 101.727 96.3422) (end 101.1936 96.8756) (width 1) (layer B.Cu) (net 11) (status 30))
 (segment (start 101.727 93.6244) (end 101.727 96.3422) (width 1) (layer B.Cu) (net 11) (status 30))
 (segment (start 96.969013 82.9564) (end 129.8956 82.9564) (width 1) (layer B.Cu) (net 12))
 (segment (start 91.355613 88.5698) (end 96.969013 82.9564) (width 1) (layer B.Cu) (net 12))
 (segment (start 89.9414 88.5698) (end 91.355613 88.5698) (width 1) (layer B.Cu) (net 12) (status 10))
 (segment (start 139.954 84.836) (end 141.1588 83.6312) (width 1) (layer B.Cu) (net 12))
 (segment (start 131.7752 84.836) (end 139.954 84.836) (width 1) (layer B.Cu) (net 12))
 (segment (start 141.1588 83.6312) (end 141.1588 82.2452) (width 1) (layer B.Cu) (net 12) (status 20))
 (segment (start 129.8956 82.9564) (end 131.7752 84.836) (width 1) (layer B.Cu) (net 12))
 (segment (start 66.7004 82.8802) (end 66.421 82.6008) (width 1) (layer B.Cu) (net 13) (status 30))
 (segment (start 66.7004 89.3318) (end 66.7004 82.8802) (width 1) (layer B.Cu) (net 13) (status 30))
 (segment (start 66.7004 96.9518) (end 69.2404 96.9518) (width 1) (layer B.Cu) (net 14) (status 30))
 (segment (start 86.969076 106.30521) (end 145.68819 106.30521) (width 1) (layer B.Cu) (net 15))
 (segment (start 82.8802 104.0638) (end 82.898866 104.0638) (width 1) (layer B.Cu) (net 15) (status 30))
 (segment (start 146.6088 105.3846) (end 146.6088 82.2452) (width 1) (layer B.Cu) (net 15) (status 20))
 (segment (start 145.68819 106.30521) (end 146.6088 105.3846) (width 1) (layer B.Cu) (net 15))
 (segment (start 82.8802 106.2638) (end 82.89 106.2736) (width 1) (layer B.Cu) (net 15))
 (segment (start 82.8802 104.0638) (end 82.8802 106.2638) (width 1) (layer B.Cu) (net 15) (status 10))
 (segment (start 86.937466 106.2736) (end 86.969076 106.30521) (width 1) (layer B.Cu) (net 15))
 (segment (start 82.89 106.2736) (end 86.937466 106.2736) (width 1) (layer B.Cu) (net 15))
 (segment (start 84.5566 82.2706) (end 79.6544 82.2706) (width 1) (layer B.Cu) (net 10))
 (segment (start 85.4202 83.1342) (end 84.5566 82.2706) (width 1) (layer B.Cu) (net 10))
 (segment (start 85.8774 93.8784) (end 85.4202 93.4212) (width 1) (layer B.Cu) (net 10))
 (segment (start 93.9546 93.8784) (end 85.8774 93.8784) (width 1) (layer B.Cu) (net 10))
 (segment (start 85.4202 93.4212) (end 85.4202 83.1342) (width 1) (layer B.Cu) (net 10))
 (segment (start 85.4202 96.4438) (end 85.4202 93.4212) (width 1) (layer B.Cu) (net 10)))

